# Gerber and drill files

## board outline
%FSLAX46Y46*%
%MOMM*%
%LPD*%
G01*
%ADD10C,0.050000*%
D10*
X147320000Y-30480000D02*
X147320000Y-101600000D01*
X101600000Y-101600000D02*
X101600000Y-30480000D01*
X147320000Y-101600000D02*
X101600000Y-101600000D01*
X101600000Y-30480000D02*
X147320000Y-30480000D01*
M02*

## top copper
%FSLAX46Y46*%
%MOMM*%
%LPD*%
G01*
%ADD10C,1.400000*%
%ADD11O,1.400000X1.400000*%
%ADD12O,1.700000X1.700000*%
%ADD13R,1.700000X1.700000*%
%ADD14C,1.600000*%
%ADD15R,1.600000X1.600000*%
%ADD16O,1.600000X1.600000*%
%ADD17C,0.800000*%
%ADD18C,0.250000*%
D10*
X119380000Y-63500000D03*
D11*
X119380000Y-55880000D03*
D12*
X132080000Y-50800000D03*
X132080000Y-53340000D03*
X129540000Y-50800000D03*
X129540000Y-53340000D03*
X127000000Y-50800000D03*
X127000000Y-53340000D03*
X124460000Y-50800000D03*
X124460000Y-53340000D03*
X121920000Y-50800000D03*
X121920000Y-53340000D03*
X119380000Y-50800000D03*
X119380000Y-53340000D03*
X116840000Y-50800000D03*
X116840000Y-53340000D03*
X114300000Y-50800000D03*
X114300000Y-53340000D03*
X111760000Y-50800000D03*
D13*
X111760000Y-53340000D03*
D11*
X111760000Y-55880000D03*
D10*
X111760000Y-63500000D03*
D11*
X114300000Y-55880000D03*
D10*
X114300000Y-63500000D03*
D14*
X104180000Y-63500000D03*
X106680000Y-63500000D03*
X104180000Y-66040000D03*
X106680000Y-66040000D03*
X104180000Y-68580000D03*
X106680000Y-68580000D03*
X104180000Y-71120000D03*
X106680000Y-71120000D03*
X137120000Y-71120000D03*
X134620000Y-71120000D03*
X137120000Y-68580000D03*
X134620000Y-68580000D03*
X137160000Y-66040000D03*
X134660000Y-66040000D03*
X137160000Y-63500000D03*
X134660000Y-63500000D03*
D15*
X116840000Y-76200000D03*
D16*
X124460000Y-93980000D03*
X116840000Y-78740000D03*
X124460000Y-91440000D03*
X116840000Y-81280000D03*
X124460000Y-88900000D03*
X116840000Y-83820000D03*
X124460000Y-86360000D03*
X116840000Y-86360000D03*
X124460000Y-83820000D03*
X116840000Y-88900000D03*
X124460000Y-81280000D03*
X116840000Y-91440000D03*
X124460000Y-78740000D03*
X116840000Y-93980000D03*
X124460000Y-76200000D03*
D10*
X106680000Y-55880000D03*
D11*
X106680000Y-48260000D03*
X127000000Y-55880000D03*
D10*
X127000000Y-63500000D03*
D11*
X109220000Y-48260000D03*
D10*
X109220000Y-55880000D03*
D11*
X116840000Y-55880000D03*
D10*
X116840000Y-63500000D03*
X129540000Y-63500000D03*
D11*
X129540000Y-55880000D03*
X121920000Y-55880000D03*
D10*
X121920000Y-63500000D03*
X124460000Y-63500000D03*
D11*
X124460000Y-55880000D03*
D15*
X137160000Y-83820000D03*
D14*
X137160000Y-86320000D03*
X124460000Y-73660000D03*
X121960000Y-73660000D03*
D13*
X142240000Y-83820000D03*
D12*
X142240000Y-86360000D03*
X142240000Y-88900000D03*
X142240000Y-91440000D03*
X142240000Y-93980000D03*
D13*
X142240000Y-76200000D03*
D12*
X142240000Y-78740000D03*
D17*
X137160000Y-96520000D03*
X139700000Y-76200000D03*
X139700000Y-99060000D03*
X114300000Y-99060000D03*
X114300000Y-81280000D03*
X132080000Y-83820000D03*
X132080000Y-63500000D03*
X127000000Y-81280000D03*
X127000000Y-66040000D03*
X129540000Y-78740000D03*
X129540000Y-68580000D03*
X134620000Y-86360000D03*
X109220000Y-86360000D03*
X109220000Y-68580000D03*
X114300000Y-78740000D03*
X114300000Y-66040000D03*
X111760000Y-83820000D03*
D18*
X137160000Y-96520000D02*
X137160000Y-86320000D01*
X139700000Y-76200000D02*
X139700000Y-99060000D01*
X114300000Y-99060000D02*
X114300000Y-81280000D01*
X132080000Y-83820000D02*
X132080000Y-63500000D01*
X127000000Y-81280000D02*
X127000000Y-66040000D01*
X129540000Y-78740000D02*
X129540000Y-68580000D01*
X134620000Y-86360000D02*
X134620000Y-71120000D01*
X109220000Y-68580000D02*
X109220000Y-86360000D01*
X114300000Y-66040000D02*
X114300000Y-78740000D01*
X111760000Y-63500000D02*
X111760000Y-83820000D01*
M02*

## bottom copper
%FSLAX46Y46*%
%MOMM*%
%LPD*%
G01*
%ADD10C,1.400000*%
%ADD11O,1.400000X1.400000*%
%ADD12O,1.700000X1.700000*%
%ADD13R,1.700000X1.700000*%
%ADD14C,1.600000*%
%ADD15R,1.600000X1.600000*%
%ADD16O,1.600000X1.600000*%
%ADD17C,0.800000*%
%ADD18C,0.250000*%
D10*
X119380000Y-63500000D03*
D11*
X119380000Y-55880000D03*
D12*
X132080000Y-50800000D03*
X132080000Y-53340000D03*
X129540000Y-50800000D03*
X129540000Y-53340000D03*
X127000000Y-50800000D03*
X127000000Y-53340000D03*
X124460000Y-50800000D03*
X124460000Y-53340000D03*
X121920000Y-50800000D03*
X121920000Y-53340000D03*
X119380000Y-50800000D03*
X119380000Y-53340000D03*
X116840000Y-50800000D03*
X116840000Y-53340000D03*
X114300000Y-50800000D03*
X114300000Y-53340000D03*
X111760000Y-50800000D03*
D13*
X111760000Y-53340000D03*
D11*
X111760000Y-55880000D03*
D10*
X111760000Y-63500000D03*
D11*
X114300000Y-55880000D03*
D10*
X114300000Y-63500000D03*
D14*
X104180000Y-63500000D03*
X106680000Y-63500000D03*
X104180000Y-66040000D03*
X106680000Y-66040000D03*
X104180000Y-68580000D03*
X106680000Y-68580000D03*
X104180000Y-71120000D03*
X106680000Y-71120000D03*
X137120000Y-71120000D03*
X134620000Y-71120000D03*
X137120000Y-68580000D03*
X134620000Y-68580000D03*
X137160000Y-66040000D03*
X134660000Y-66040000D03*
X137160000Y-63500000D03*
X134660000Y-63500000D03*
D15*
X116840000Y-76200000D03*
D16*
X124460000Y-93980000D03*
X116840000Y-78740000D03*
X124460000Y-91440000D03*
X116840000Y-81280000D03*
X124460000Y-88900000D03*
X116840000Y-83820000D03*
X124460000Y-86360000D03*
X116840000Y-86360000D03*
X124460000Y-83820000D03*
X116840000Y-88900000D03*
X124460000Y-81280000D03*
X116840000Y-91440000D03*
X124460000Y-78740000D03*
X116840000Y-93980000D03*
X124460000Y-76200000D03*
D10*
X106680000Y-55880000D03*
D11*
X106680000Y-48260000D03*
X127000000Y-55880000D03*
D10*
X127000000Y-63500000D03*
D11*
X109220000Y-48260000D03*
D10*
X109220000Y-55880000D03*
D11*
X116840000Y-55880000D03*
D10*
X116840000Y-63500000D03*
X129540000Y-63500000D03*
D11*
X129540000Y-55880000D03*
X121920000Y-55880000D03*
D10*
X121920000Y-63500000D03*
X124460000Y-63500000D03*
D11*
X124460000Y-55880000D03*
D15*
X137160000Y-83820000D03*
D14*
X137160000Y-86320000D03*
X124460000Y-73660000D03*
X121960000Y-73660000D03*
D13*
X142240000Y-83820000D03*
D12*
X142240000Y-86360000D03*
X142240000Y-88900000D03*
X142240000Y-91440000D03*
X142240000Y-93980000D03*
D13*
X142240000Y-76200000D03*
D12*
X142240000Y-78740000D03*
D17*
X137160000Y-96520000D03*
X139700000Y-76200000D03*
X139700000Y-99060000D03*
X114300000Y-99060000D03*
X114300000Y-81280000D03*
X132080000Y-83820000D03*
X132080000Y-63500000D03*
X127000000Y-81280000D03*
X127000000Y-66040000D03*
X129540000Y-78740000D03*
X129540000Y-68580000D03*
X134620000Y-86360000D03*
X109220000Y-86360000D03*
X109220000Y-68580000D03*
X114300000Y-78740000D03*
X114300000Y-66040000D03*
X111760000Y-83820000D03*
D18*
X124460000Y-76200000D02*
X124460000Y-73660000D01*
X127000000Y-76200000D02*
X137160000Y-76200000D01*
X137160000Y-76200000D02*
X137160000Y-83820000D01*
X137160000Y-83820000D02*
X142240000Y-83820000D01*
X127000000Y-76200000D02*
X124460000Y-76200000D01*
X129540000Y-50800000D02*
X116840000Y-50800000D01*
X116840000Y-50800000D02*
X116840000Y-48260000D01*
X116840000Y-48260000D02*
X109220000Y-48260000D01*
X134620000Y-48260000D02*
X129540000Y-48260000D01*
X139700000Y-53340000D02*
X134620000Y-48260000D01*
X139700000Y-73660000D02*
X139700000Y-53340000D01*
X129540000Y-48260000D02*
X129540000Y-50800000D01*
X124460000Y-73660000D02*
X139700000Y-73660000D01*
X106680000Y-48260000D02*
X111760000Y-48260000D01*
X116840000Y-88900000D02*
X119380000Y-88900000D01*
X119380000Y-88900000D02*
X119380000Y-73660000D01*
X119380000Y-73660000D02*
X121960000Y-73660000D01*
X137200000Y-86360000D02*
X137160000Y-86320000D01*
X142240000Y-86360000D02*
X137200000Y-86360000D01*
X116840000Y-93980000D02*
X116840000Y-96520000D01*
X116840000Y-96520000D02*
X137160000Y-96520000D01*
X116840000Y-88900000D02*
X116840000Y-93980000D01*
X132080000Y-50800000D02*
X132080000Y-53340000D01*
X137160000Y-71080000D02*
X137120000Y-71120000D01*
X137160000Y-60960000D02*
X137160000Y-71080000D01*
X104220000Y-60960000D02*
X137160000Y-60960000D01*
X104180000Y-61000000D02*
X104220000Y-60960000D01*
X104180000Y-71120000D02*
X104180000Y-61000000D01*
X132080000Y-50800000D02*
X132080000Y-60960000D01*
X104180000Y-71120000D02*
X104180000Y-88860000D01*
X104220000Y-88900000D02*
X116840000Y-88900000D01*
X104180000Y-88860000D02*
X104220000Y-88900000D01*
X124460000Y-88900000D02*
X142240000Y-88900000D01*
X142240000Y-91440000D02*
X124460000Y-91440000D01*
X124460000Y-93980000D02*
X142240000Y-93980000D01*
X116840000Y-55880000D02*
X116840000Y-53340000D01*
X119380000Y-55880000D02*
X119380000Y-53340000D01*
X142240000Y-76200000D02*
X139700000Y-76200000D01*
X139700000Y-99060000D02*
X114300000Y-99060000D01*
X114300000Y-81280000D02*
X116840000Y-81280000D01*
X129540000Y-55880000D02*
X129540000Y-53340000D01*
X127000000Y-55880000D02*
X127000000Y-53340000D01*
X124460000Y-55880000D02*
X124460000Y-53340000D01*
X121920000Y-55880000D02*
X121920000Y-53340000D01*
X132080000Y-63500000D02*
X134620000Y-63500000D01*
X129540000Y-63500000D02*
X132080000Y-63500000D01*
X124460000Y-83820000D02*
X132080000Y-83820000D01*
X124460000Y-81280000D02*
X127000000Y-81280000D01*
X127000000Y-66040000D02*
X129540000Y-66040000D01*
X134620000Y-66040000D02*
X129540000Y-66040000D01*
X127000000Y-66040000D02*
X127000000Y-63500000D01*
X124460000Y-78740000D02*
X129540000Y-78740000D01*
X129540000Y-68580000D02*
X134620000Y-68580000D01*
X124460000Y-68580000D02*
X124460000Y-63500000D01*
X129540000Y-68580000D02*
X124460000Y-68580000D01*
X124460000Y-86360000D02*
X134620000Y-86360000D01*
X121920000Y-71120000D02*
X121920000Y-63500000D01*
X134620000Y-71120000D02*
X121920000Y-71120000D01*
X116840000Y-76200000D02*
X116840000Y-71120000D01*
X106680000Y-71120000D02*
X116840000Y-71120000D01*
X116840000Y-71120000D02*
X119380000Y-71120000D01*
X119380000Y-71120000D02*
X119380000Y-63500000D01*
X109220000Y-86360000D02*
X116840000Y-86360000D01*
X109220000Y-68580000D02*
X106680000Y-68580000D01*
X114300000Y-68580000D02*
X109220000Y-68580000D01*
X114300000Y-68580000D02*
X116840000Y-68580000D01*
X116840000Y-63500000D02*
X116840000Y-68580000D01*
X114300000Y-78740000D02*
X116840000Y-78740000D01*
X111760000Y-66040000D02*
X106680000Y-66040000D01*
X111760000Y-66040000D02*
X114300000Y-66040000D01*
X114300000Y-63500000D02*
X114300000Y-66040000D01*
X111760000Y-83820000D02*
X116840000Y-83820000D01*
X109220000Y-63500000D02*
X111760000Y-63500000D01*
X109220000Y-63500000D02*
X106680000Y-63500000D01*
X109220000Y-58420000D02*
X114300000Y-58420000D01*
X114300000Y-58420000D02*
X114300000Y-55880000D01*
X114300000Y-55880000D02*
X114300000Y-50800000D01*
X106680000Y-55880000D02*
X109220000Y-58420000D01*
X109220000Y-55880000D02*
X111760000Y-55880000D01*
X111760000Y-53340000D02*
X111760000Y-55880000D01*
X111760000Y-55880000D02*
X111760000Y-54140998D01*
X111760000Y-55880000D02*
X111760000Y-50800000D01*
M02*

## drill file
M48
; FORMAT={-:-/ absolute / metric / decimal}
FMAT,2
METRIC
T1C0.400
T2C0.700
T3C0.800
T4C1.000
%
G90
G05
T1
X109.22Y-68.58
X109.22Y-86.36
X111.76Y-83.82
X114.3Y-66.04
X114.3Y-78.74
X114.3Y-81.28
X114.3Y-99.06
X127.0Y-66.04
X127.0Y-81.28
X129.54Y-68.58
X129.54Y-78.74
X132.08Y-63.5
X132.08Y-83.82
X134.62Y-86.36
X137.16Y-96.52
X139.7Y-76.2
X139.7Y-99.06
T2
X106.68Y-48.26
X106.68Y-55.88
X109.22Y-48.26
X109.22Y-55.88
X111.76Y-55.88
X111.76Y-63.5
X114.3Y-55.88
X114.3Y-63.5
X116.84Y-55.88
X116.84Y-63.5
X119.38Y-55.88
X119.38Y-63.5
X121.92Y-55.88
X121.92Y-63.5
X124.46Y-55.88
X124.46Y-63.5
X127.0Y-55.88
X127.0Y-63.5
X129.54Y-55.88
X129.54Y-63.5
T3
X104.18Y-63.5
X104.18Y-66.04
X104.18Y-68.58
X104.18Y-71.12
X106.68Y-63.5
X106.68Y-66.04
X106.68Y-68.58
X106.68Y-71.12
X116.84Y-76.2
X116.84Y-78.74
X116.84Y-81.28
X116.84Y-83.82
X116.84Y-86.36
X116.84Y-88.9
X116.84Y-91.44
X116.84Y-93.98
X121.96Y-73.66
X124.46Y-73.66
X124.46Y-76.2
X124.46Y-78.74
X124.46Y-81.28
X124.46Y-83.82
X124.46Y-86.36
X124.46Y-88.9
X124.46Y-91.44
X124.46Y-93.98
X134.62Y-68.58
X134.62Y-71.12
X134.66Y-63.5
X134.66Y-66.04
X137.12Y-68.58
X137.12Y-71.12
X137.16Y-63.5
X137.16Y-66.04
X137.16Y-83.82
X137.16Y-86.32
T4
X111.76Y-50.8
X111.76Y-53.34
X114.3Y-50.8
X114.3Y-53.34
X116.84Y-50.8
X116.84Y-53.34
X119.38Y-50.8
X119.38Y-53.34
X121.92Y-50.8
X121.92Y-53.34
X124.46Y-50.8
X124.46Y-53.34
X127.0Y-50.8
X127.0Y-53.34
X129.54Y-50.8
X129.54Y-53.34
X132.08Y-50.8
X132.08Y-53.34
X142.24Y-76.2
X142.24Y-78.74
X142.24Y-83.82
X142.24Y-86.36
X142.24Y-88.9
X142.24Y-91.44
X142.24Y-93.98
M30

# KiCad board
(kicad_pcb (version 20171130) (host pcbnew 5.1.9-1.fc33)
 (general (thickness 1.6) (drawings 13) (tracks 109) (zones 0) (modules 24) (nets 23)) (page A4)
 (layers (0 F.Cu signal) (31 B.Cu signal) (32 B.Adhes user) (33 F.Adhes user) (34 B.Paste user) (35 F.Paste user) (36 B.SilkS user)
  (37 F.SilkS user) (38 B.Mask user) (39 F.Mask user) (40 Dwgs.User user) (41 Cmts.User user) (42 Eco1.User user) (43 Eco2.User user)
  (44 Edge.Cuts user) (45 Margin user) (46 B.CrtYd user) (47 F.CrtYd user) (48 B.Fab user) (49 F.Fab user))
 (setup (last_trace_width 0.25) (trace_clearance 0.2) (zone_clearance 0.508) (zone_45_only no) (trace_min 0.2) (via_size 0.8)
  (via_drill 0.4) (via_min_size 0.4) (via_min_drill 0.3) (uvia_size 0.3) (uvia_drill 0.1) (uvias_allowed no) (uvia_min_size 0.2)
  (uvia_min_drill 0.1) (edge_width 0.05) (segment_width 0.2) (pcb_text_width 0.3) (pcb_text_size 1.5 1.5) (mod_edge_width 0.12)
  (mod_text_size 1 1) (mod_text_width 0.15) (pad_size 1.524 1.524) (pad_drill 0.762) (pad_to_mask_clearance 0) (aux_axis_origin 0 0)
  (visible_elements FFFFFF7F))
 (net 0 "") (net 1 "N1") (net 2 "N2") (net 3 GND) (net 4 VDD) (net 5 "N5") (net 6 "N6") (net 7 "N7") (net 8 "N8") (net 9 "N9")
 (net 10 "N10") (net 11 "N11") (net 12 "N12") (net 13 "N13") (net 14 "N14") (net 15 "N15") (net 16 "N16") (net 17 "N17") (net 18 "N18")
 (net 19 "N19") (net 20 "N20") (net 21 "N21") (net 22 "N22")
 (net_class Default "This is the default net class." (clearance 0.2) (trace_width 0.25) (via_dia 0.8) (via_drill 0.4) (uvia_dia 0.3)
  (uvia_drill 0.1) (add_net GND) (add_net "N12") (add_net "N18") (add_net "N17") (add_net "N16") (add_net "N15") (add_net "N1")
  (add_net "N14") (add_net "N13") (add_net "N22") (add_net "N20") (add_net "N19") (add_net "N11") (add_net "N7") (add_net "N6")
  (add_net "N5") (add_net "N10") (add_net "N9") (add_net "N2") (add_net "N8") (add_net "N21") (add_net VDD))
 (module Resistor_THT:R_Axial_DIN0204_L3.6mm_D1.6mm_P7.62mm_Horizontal (layer F.Cu) (at 119.38 63.5 90)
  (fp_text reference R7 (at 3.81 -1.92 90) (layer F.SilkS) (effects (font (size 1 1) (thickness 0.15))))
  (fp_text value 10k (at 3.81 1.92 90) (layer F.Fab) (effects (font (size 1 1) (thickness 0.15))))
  (pad 1 thru_hole circle (at 0 0 90) (size 1.4 1.4) (drill 0.7) (layers *.Cu *.Mask) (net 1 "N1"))
  (pad 2 thru_hole oval (at 7.62 0 90) (size 1.4 1.4) (drill 0.7) (layers *.Cu *.Mask) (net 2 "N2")))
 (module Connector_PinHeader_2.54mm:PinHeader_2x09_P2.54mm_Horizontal (layer F.Cu) (at 111.76 53.34 90)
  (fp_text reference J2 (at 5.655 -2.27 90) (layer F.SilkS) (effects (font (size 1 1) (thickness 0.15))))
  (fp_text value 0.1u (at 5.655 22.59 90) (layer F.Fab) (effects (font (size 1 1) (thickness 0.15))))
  (pad 18 thru_hole oval (at 2.54 20.32 90) (size 1.7 1.7) (drill 1) (layers *.Cu *.Mask) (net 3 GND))
  (pad 17 thru_hole oval (at 0 20.32 90) (size 1.7 1.7) (drill 1) (layers *.Cu *.Mask) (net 3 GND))
  (pad 16 thru_hole oval (at 2.54 17.78 90) (size 1.7 1.7) (drill 1) (layers *.Cu *.Mask) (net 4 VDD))
  (pad 15 thru_hole oval (at 0 17.78 90) (size 1.7 1.7) (drill 1) (layers *.Cu *.Mask) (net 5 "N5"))
  (pad 14 thru_hole oval (at 2.54 15.24 90) (size 1.7 1.7) (drill 1) (layers *.Cu *.Mask) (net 4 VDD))
  (pad 13 thru_hole oval (at 0 15.24 90) (size 1.7 1.7) (drill 1) (layers *.Cu *.Mask) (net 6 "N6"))
  (pad 12 thru_hole oval (at 2.54 12.7 90) (size 1.7 1.7) (drill 1) (layers *.Cu *.Mask) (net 4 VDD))
  (pad 11 thru_hole oval (at 0 12.7 90) (size 1.7 1.7) (drill 1) (layers *.Cu *.Mask) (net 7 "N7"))
  (pad 10 thru_hole oval (at 2.54 10.16 90) (size 1.7 1.7) (drill 1) (layers *.Cu *.Mask) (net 4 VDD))
  (pad 9 thru_hole oval (at 0 10.16 90) (size 1.7 1.7) (drill 1) (layers *.Cu *.Mask) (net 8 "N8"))
  (pad 8 thru_hole oval (at 2.54 7.62 90) (size 1.7 1.7) (drill 1) (layers *.Cu *.Mask) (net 4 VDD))
  (pad 7 thru_hole oval (at 0 7.62 90) (size 1.7 1.7) (drill 1) (layers *.Cu *.Mask) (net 2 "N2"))
  (pad 6 thru_hole oval (at 2.54 5.08 90) (size 1.7 1.7) (drill 1) (layers *.Cu *.Mask) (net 4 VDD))
  (pad 5 thru_hole oval (at 0 5.08 90) (size 1.7 1.7) (drill 1) (layers *.Cu *.Mask) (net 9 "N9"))
  (pad 4 thru_hole oval (at 2.54 2.54 90) (size 1.7 1.7) (drill 1) (layers *.Cu *.Mask) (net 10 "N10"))
  (pad 3 thru_hole oval (at 0 2.54 90) (size 1.7 1.7) (drill 1) (layers *.Cu *.Mask) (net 10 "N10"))
  (pad 2 thru_hole oval (at 2.54 0 90) (size 1.7 1.7) (drill 1) (layers *.Cu *.Mask) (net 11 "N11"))
  (pad 1 thru_hole rect (at 0 0 90) (size 1.7 1.7) (drill 1) (layers *.Cu *.Mask) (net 11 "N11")))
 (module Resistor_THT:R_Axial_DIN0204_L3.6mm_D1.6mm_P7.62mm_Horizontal (layer F.Cu) (at 111.76 63.5 90)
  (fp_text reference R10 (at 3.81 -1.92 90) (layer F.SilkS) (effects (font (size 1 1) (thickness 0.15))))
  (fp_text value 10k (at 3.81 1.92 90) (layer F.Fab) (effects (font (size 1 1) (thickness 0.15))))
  (pad 2 thru_hole oval (at 7.62 0 90) (size 1.4 1.4) (drill 0.7) (layers *.Cu *.Mask) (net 11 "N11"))
  (pad 1 thru_hole circle (at 0 0 90) (size 1.4 1.4) (drill 0.7) (layers *.Cu *.Mask) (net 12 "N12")))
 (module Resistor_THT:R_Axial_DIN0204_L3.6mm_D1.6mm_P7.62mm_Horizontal (layer F.Cu) (at 114.3 63.5 90)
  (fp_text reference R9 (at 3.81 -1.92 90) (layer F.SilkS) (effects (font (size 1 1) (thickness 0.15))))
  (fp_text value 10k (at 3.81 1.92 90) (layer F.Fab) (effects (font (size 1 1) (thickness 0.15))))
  (pad 2 thru_hole oval (at 7.62 0 90) (size 1.4 1.4) (drill 0.7) (layers *.Cu *.Mask) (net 10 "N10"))
  (pad 1 thru_hole circle (at 0 0 90) (size 1.4 1.4) (drill 0.7) (layers *.Cu *.Mask) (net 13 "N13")))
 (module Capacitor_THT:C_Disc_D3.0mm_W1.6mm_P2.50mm (layer F.Cu) (at 106.68 63.5 180)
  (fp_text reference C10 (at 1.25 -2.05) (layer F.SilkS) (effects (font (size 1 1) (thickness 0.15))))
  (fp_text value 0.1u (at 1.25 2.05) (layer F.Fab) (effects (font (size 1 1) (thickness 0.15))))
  (pad 2 thru_hole circle (at 2.5 0 180) (size 1.6 1.6) (drill 0.8) (layers *.Cu *.Mask) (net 3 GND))
  (pad 1 thru_hole circle (at 0 0 180) (size 1.6 1.6) (drill 0.8) (layers *.Cu *.Mask) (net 12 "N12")))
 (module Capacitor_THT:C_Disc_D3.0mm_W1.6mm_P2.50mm (layer F.Cu) (at 106.68 66.04 180)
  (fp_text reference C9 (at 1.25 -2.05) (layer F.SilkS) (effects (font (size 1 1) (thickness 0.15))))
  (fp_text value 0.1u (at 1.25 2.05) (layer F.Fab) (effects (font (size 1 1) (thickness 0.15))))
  (pad 2 thru_hole circle (at 2.5 0 180) (size 1.6 1.6) (drill 0.8) (layers *.Cu *.Mask) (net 3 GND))
  (pad 1 thru_hole circle (at 0 0 180) (size 1.6 1.6) (drill 0.8) (layers *.Cu *.Mask) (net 13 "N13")))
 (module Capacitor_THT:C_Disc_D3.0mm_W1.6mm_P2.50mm (layer F.Cu) (at 106.68 68.58 180)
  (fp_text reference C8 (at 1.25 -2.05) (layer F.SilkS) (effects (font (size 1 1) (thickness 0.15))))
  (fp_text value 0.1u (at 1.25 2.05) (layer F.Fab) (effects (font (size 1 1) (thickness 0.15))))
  (pad 2 thru_hole circle (at 2.5 0 180) (size 1.6 1.6) (drill 0.8) (layers *.Cu *.Mask) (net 3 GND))
  (pad 1 thru_hole circle (at 0 0 180) (size 1.6 1.6) (drill 0.8) (layers *.Cu *.Mask) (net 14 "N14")))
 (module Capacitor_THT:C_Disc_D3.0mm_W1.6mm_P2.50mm (layer F.Cu) (at 106.68 71.12 180)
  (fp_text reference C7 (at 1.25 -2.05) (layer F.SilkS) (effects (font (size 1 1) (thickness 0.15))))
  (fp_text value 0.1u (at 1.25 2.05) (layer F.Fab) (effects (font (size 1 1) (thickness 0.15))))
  (pad 2 thru_hole circle (at 2.5 0 180) (size 1.6 1.6) (drill 0.8) (layers *.Cu *.Mask) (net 3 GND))
  (pad 1 thru_hole circle (at 0 0 180) (size 1.6 1.6) (drill 0.8) (layers *.Cu *.Mask) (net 1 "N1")))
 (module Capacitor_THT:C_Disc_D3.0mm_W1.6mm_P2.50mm (layer F.Cu) (at 134.62 71.12)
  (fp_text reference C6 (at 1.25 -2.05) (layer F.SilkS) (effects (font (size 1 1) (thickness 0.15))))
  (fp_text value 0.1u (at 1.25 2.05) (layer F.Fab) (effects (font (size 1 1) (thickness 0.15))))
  (pad 2 thru_hole circle (at 2.5 0) (size 1.6 1.6) (drill 0.8) (layers *.Cu *.Mask) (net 3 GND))
  (pad 1 thru_hole circle (at 0 0) (size 1.6 1.6) (drill 0.8) (layers *.Cu *.Mask) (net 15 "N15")))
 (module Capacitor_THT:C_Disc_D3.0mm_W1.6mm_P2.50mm (layer F.Cu) (at 134.62 68.58)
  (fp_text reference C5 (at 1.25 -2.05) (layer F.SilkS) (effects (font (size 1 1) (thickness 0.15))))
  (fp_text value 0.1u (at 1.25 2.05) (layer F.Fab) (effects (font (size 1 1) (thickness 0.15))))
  (pad 2 thru_hole circle (at 2.5 0) (size 1.6 1.6) (drill 0.8) (layers *.Cu *.Mask) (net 3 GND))
  (pad 1 thru_hole circle (at 0 0) (size 1.6 1.6) (drill 0.8) (layers *.Cu *.Mask) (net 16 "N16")))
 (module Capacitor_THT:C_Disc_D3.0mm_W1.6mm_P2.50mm (layer F.Cu) (at 134.66 66.04)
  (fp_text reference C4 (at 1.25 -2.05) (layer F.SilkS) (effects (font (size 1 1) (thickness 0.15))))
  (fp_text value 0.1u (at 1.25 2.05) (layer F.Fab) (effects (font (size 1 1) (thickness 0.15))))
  (pad 2 thru_hole circle (at 2.5 0) (size 1.6 1.6) (drill 0.8) (layers *.Cu *.Mask) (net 3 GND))
  (pad 1 thru_hole circle (at 0 0) (size 1.6 1.6) (drill 0.8) (layers *.Cu *.Mask) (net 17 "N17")))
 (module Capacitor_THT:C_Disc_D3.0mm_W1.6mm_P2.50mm (layer F.Cu) (at 134.66 63.5)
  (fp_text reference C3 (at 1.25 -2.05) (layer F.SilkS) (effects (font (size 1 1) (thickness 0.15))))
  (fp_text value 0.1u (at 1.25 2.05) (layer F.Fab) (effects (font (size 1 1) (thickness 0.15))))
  (pad 2 thru_hole circle (at 2.5 0) (size 1.6 1.6) (drill 0.8) (layers *.Cu *.Mask) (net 3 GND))
  (pad 1 thru_hole circle (at 0 0) (size 1.6 1.6) (drill 0.8) (layers *.Cu *.Mask) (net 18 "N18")))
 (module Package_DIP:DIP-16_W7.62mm (layer F.Cu) (at 116.84 76.2)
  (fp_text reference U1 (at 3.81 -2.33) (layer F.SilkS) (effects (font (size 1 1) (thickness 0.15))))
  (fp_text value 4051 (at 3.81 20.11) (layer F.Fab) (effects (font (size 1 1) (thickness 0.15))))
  (pad 1 thru_hole rect (at 0 0) (size 1.6 1.6) (drill 0.8) (layers *.Cu *.Mask) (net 1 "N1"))
  (pad 9 thru_hole oval (at 7.62 17.78) (size 1.6 1.6) (drill 0.8) (layers *.Cu *.Mask) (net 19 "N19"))
  (pad 2 thru_hole oval (at 0 2.54) (size 1.6 1.6) (drill 0.8) (layers *.Cu *.Mask) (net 13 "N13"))
  (pad 10 thru_hole oval (at 7.62 15.24) (size 1.6 1.6) (drill 0.8) (layers *.Cu *.Mask) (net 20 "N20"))
  (pad 3 thru_hole oval (at 0 5.08) (size 1.6 1.6) (drill 0.8) (layers *.Cu *.Mask) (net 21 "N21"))
  (pad 11 thru_hole oval (at 7.62 12.7) (size 1.6 1.6) (drill 0.8) (layers *.Cu *.Mask) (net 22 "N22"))
  (pad 4 thru_hole oval (at 0 7.62) (size 1.6 1.6) (drill 0.8) (layers *.Cu *.Mask) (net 12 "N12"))
  (pad 12 thru_hole oval (at 7.62 10.16) (size 1.6 1.6) (drill 0.8) (layers *.Cu *.Mask) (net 15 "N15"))
  (pad 5 thru_hole oval (at 0 10.16) (size 1.6 1.6) (drill 0.8) (layers *.Cu *.Mask) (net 14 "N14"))
  (pad 13 thru_hole oval (at 7.62 7.62) (size 1.6 1.6) (drill 0.8) (layers *.Cu *.Mask) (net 18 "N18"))
  (pad 6 thru_hole oval (at 0 12.7) (size 1.6 1.6) (drill 0.8) (layers *.Cu *.Mask) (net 3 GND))
  (pad 14 thru_hole oval (at 7.62 5.08) (size 1.6 1.6) (drill 0.8) (layers *.Cu *.Mask) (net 17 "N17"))
  (pad 7 thru_hole oval (at 0 15.24) (size 1.6 1.6) (drill 0.8) (layers *.Cu *.Mask) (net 3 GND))
  (pad 15 thru_hole oval (at 7.62 2.54) (size 1.6 1.6) (drill 0.8) (layers *.Cu *.Mask) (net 16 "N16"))
  (pad 8 thru_hole oval (at 0 17.78) (size 1.6 1.6) (drill 0.8) (layers *.Cu *.Mask) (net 3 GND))
  (pad 16 thru_hole oval (at 7.62 0) (size 1.6 1.6) (drill 0.8) (layers *.Cu *.Mask) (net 4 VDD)))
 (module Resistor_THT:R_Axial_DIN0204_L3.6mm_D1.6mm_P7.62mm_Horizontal (layer F.Cu) (at 106.68 55.88 90)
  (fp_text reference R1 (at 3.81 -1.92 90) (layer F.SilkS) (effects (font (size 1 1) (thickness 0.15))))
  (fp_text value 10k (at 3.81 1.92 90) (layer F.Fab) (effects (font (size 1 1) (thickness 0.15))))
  (pad 1 thru_hole circle (at 0 0 90) (size 1.4 1.4) (drill 0.7) (layers *.Cu *.Mask) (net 10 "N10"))
  (pad 2 thru_hole oval (at 7.62 0 90) (size 1.4 1.4) (drill 0.7) (layers *.Cu *.Mask) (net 4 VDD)))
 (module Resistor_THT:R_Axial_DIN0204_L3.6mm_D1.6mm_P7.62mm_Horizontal (layer F.Cu) (at 127 63.5 90)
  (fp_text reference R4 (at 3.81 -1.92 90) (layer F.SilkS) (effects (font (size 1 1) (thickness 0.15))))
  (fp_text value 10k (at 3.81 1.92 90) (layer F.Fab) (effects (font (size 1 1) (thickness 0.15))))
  (pad 2 thru_hole oval (at 7.62 0 90) (size 1.4 1.4) (drill 0.7) (layers *.Cu *.Mask) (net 6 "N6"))
  (pad 1 thru_hole circle (at 0 0 90) (size 1.4 1.4) (drill 0.7) (layers *.Cu *.Mask) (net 17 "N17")))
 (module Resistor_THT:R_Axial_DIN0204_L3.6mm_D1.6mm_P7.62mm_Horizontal (layer F.Cu) (at 109.22 55.88 90)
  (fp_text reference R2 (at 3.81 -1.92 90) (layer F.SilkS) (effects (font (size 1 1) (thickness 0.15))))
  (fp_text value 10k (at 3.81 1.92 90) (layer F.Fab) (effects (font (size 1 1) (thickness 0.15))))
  (pad 2 thru_hole oval (at 7.62 0 90) (size 1.4 1.4) (drill 0.7) (layers *.Cu *.Mask) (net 4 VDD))
  (pad 1 thru_hole circle (at 0 0 90) (size 1.4 1.4) (drill 0.7) (layers *.Cu *.Mask) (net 11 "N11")))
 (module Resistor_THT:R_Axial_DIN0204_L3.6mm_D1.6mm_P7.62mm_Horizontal (layer F.Cu) (at 116.84 63.5 90)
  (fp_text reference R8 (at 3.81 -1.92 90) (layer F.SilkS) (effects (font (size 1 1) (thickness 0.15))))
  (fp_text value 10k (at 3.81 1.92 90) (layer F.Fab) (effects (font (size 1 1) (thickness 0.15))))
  (pad 2 thru_hole oval (at 7.62 0 90) (size 1.4 1.4) (drill 0.7) (layers *.Cu *.Mask) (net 9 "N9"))
  (pad 1 thru_hole circle (at 0 0 90) (size 1.4 1.4) (drill 0.7) (layers *.Cu *.Mask) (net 14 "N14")))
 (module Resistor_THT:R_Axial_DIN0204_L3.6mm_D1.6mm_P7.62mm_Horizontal (layer F.Cu) (at 129.54 63.5 90)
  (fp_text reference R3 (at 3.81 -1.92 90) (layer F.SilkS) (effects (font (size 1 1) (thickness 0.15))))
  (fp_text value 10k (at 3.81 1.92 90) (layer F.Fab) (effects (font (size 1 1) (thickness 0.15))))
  (pad 1 thru_hole circle (at 0 0 90) (size 1.4 1.4) (drill 0.7) (layers *.Cu *.Mask) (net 18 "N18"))
  (pad 2 thru_hole oval (at 7.62 0 90) (size 1.4 1.4) (drill 0.7) (layers *.Cu *.Mask) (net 5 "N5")))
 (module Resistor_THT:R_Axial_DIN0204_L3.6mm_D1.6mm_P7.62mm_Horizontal (layer F.Cu) (at 121.92 63.5 90)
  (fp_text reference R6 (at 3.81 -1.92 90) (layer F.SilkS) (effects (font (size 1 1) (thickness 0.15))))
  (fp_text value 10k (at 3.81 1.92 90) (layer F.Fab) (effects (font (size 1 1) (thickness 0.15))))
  (pad 2 thru_hole oval (at 7.62 0 90) (size 1.4 1.4) (drill 0.7) (layers *.Cu *.Mask) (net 8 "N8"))
  (pad 1 thru_hole circle (at 0 0 90) (size 1.4 1.4) (drill 0.7) (layers *.Cu *.Mask) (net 15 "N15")))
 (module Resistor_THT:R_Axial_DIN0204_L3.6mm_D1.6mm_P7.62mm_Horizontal (layer F.Cu) (at 124.46 63.5 90)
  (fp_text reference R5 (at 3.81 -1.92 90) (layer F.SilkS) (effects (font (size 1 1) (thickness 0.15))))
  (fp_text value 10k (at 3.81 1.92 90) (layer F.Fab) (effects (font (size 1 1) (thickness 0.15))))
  (pad 1 thru_hole circle (at 0 0 90) (size 1.4 1.4) (drill 0.7) (layers *.Cu *.Mask) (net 16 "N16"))
  (pad 2 thru_hole oval (at 7.62 0 90) (size 1.4 1.4) (drill 0.7) (layers *.Cu *.Mask) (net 7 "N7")))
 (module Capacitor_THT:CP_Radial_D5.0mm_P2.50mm (layer F.Cu) (at 137.16 83.82 270)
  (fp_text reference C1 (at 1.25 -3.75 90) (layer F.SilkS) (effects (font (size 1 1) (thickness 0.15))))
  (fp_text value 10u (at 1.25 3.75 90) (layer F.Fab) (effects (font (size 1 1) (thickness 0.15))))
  (pad 1 thru_hole rect (at 0 0 270) (size 1.6 1.6) (drill 0.8) (layers *.Cu *.Mask) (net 4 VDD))
  (pad 2 thru_hole circle (at 2.5 0 270) (size 1.6 1.6) (drill 0.8) (layers *.Cu *.Mask) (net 3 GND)))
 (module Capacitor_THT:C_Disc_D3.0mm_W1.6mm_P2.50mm (layer F.Cu) (at 124.46 73.66 180)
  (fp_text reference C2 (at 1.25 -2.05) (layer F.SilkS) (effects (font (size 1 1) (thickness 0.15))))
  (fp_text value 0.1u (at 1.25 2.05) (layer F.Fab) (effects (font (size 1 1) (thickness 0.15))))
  (pad 1 thru_hole circle (at 0 0 180) (size 1.6 1.6) (drill 0.8) (layers *.Cu *.Mask) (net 4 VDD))
  (pad 2 thru_hole circle (at 2.5 0 180) (size 1.6 1.6) (drill 0.8) (layers *.Cu *.Mask) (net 3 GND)))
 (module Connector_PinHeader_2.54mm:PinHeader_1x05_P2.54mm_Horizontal (layer F.Cu) (at 142.24 83.82)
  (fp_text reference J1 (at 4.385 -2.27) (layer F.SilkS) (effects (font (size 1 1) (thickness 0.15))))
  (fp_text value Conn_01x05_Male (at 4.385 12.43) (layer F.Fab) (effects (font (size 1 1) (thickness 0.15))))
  (pad 1 thru_hole rect (at 0 0) (size 1.7 1.7) (drill 1) (layers *.Cu *.Mask) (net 4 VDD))
  (pad 2 thru_hole oval (at 0 2.54) (size 1.7 1.7) (drill 1) (layers *.Cu *.Mask) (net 3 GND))
  (pad 3 thru_hole oval (at 0 5.08) (size 1.7 1.7) (drill 1) (layers *.Cu *.Mask) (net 22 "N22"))
  (pad 4 thru_hole oval (at 0 7.62) (size 1.7 1.7) (drill 1) (layers *.Cu *.Mask) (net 20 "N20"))
  (pad 5 thru_hole oval (at 0 10.16) (size 1.7 1.7) (drill 1) (layers *.Cu *.Mask) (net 19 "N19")))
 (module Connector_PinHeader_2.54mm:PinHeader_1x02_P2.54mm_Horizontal (layer F.Cu) (at 142.24 76.2)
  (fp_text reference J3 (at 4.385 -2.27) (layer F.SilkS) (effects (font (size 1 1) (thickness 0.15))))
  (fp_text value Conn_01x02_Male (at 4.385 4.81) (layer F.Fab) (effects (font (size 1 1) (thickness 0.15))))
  (pad 1 thru_hole rect (at 0 0) (size 1.7 1.7) (drill 1) (layers *.Cu *.Mask) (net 21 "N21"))
  (pad 2 thru_hole oval (at 0 2.54) (size 1.7 1.7) (drill 1) (layers *.Cu *.Mask)))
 (gr_line (start 147.32 30.48) (end 147.32 101.6) (layer Edge.Cuts) (width 0.05))
 (gr_line (start 101.6 101.6) (end 101.6 30.48) (layer Edge.Cuts) (width 0.05))
 (gr_line (start 147.32 101.6) (end 101.6 101.6) (layer Edge.Cuts) (width 0.05))
 (gr_line (start 101.6 30.48) (end 147.32 30.48) (layer Edge.Cuts) (width 0.05))
 (segment (start 124.46 76.2) (end 124.46 73.66) (width 0.25) (layer B.Cu) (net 4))
 (segment (start 127 76.2) (end 137.16 76.2) (width 0.25) (layer B.Cu) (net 4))
 (segment (start 137.16 76.2) (end 137.16 83.82) (width 0.25) (layer B.Cu) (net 4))
 (segment (start 137.16 83.82) (end 142.24 83.82) (width 0.25) (layer B.Cu) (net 4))
 (segment (start 127 76.2) (end 124.46 76.2) (width 0.25) (layer B.Cu) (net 4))
 (segment (start 129.54 50.8) (end 116.84 50.8) (width 0.25) (layer B.Cu) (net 4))
 (segment (start 116.84 50.8) (end 116.84 48.26) (width 0.25) (layer B.Cu) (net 4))
 (segment (start 116.84 48.26) (end 109.22 48.26) (width 0.25) (layer B.Cu) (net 4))
 (segment (start 134.62 48.26) (end 129.54 48.26) (width 0.25) (layer B.Cu) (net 4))
 (segment (start 139.7 53.34) (end 134.62 48.26) (width 0.25) (layer B.Cu) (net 4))
 (segment (start 139.7 73.66) (end 139.7 53.34) (width 0.25) (layer B.Cu) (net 4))
 (segment (start 129.54 48.26) (end 129.54 50.8) (width 0.25) (layer B.Cu) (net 4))
 (segment (start 124.46 73.66) (end 139.7 73.66) (width 0.25) (layer B.Cu) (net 4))
 (segment (start 106.68 48.26) (end 111.76 48.26) (width 0.25) (layer B.Cu) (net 4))
 (segment (start 116.84 88.9) (end 119.38 88.9) (width 0.25) (layer B.Cu) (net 3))
 (segment (start 119.38 88.9) (end 119.38 73.66) (width 0.25) (layer B.Cu) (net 3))
 (segment (start 119.38 73.66) (end 121.96 73.66) (width 0.25) (layer B.Cu) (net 3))
 (segment (start 137.2 86.36) (end 137.16 86.32) (width 0.25) (layer B.Cu) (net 3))
 (segment (start 142.24 86.36) (end 137.2 86.36) (width 0.25) (layer B.Cu) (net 3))
 (segment (start 116.84 93.98) (end 116.84 96.52) (width 0.25) (layer B.Cu) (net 3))
 (via (at 137.16 96.52) (size 0.8) (drill 0.4) (layers F.Cu B.Cu) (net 3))
 (segment (start 116.84 96.52) (end 137.16 96.52) (width 0.25) (layer B.Cu) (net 3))
 (segment (start 137.16 96.52) (end 137.16 86.32) (width 0.25) (layer F.Cu) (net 3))
 (segment (start 116.84 88.9) (end 116.84 93.98) (width 0.25) (layer B.Cu) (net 3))
 (segment (start 132.08 50.8) (end 132.08 53.34) (width 0.25) (layer B.Cu) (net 3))
 (segment (start 137.16 71.08) (end 137.12 71.12) (width 0.25) (layer B.Cu) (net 3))
 (segment (start 137.16 60.96) (end 137.16 71.08) (width 0.25) (layer B.Cu) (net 3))
 (segment (start 104.22 60.96) (end 137.16 60.96) (width 0.25) (layer B.Cu) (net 3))
 (segment (start 104.18 61) (end 104.22 60.96) (width 0.25) (layer B.Cu) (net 3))
 (segment (start 104.18 71.12) (end 104.18 61) (width 0.25) (layer B.Cu) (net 3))
 (segment (start 132.08 50.8) (end 132.08 60.96) (width 0.25) (layer B.Cu) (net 3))
 (segment (start 104.18 71.12) (end 104.18 88.86) (width 0.25) (layer B.Cu) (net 3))
 (segment (start 104.22 88.9) (end 116.84 88.9) (width 0.25) (layer B.Cu) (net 3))
 (segment (start 104.18 88.86) (end 104.22 88.9) (width 0.25) (layer B.Cu) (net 3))
 (segment (start 124.46 88.9) (end 142.24 88.9) (width 0.25) (layer B.Cu) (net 22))
 (segment (start 142.24 91.44) (end 124.46 91.44) (width 0.25) (layer B.Cu) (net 20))
 (segment (start 124.46 93.98) (end 142.24 93.98) (width 0.25) (layer B.Cu) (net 19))
 (segment (start 116.84 55.88) (end 116.84 53.34) (width 0.25) (layer B.Cu) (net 9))
 (segment (start 119.38 55.88) (end 119.38 53.34) (width 0.25) (layer B.Cu) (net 2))
 (via (at 139.7 76.2) (size 0.8) (drill 0.4) (layers F.Cu B.Cu) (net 21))
 (segment (start 142.24 76.2) (end 139.7 76.2) (width 0.25) (layer B.Cu) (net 21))
 (via (at 139.7 99.06) (size 0.8) (drill 0.4) (layers F.Cu B.Cu) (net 21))
 (segment (start 139.7 76.2) (end 139.7 99.06) (width 0.25) (layer F.Cu) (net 21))
 (via (at 114.3 99.06) (size 0.8) (drill 0.4) (layers F.Cu B.Cu) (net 21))
 (segment (start 139.7 99.06) (end 114.3 99.06) (width 0.25) (layer B.Cu) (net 21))
 (via (at 114.3 81.28) (size 0.8) (drill 0.4) (layers F.Cu B.Cu) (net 21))
 (segment (start 114.3 99.06) (end 114.3 81.28) (width 0.25) (layer F.Cu) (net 21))
 (segment (start 114.3 81.28) (end 116.84 81.28) (width 0.25) (layer B.Cu) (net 21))
 (segment (start 129.54 55.88) (end 129.54 53.34) (width 0.25) (layer B.Cu) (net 5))
 (segment (start 127 55.88) (end 127 53.34) (width 0.25) (layer B.Cu) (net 6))
 (segment (start 124.46 55.88) (end 124.46 53.34) (width 0.25) (layer B.Cu) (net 7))
 (segment (start 121.92 55.88) (end 121.92 53.34) (width 0.25) (layer B.Cu) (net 8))
 (segment (start 132.08 63.5) (end 134.62 63.5) (width 0.25) (layer B.Cu) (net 18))
 (segment (start 129.54 63.5) (end 132.08 63.5) (width 0.25) (layer B.Cu) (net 18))
 (via (at 132.08 83.82) (size 0.8) (drill 0.4) (layers F.Cu B.Cu) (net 18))
 (segment (start 124.46 83.82) (end 132.08 83.82) (width 0.25) (layer B.Cu) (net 18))
 (segment (start 132.08 83.82) (end 132.08 63.5) (width 0.25) (layer F.Cu) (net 18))
 (via (at 132.08 63.5) (size 0.8) (drill 0.4) (layers F.Cu B.Cu) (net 18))
 (via (at 127 81.28) (size 0.8) (drill 0.4) (layers F.Cu B.Cu) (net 17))
 (segment (start 124.46 81.28) (end 127 81.28) (width 0.25) (layer B.Cu) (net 17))
 (segment (start 127 66.04) (end 129.54 66.04) (width 0.25) (layer B.Cu) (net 17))
 (segment (start 134.62 66.04) (end 129.54 66.04) (width 0.25) (layer B.Cu) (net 17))
 (via (at 127 66.04) (size 0.8) (drill 0.4) (layers F.Cu B.Cu) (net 17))
 (segment (start 127 81.28) (end 127 66.04) (width 0.25) (layer F.Cu) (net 17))
 (segment (start 127 66.04) (end 127 63.5) (width 0.25) (layer B.Cu) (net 17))
 (via (at 129.54 78.74) (size 0.8) (drill 0.4) (layers F.Cu B.Cu) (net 16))
 (segment (start 124.46 78.74) (end 129.54 78.74) (width 0.25) (layer B.Cu) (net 16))
 (segment (start 129.54 68.58) (end 134.62 68.58) (width 0.25) (layer B.Cu) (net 16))
 (segment (start 129.54 78.74) (end 129.54 68.58) (width 0.25) (layer F.Cu) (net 16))
 (via (at 129.54 68.58) (size 0.8) (drill 0.4) (layers F.Cu B.Cu) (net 16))
 (segment (start 124.46 68.58) (end 124.46 63.5) (width 0.25) (layer B.Cu) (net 16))
 (segment (start 129.54 68.58) (end 124.46 68.58) (width 0.25) (layer B.Cu) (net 16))
 (segment (start 124.46 86.36) (end 134.62 86.36) (width 0.25) (layer B.Cu) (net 15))
 (via (at 134.62 86.36) (size 0.8) (drill 0.4) (layers F.Cu B.Cu) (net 15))
 (segment (start 134.62 86.36) (end 134.62 71.12) (width 0.25) (layer F.Cu) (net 15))
 (segment (start 121.92 71.12) (end 121.92 63.5) (width 0.25) (layer B.Cu) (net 15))
 (segment (start 134.62 71.12) (end 121.92 71.12) (width 0.25) (layer B.Cu) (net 15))
 (segment (start 116.84 76.2) (end 116.84 71.12) (width 0.25) (layer B.Cu) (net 1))
 (segment (start 106.68 71.12) (end 116.84 71.12) (width 0.25) (layer B.Cu) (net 1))
 (segment (start 116.84 71.12) (end 119.38 71.12) (width 0.25) (layer B.Cu) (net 1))
 (segment (start 119.38 71.12) (end 119.38 63.5) (width 0.25) (layer B.Cu) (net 1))
 (via (at 109.22 86.36) (size 0.8) (drill 0.4) (layers F.Cu B.Cu) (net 14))
 (segment (start 109.22 86.36) (end 116.84 86.36) (width 0.25) (layer B.Cu) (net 14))
 (segment (start 109.22 68.58) (end 109.22 86.36) (width 0.25) (layer F.Cu) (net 14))
 (segment (start 109.22 68.58) (end 106.68 68.58) (width 0.25) (layer B.Cu) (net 14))
 (segment (start 114.3 68.58) (end 109.22 68.58) (width 0.25) (layer B.Cu) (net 14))
 (via (at 109.22 68.58) (size 0.8) (drill 0.4) (layers F.Cu B.Cu) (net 14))
 (segment (start 114.3 68.58) (end 116.84 68.58) (width 0.25) (layer B.Cu) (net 14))
 (segment (start 116.84 63.5) (end 116.84 68.58) (width 0.25) (layer B.Cu) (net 14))
 (via (at 114.3 78.74) (size 0.8) (drill 0.4) (layers F.Cu B.Cu) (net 13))
 (segment (start 114.3 78.74) (end 116.84 78.74) (width 0.25) (layer B.Cu) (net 13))
 (segment (start 111.76 66.04) (end 106.68 66.04) (width 0.25) (layer B.Cu) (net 13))
 (segment (start 114.3 66.04) (end 114.3 78.74) (width 0.25) (layer F.Cu) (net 13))
 (via (at 114.3 66.04) (size 0.8) (drill 0.4) (layers F.Cu B.Cu) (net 13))
 (segment (start 111.76 66.04) (end 114.3 66.04) (width 0.25) (layer B.Cu) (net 13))
 (segment (start 114.3 63.5) (end 114.3 66.04) (width 0.25) (layer B.Cu) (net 13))
 (via (at 111.76 83.82) (size 0.8) (drill 0.4) (layers F.Cu B.Cu) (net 12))
 (segment (start 111.76 83.82) (end 116.84 83.82) (width 0.25) (layer B.Cu) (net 12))
 (segment (start 111.76 63.5) (end 111.76 83.82) (width 0.25) (layer F.Cu) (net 12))
 (segment (start 109.22 63.5) (end 111.76 63.5) (width 0.25) (layer B.Cu) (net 12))
 (segment (start 109.22 63.5) (end 106.68 63.5) (width 0.25) (layer B.Cu) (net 12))
 (segment (start 109.22 58.42) (end 114.3 58.42) (width 0.25) (layer B.Cu) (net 10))
 (segment (start 114.3 58.42) (end 114.3 55.88) (width 0.25) (layer B.Cu) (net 10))
 (segment (start 114.3 55.88) (end 114.3 50.8) (width 0.25) (layer B.Cu) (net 10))
 (segment (start 106.68 55.88) (end 109.22 58.42) (width 0.25) (layer B.Cu) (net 10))
 (segment (start 109.22 55.88) (end 111.76 55.88) (width 0.25) (layer B.Cu) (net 11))
 (segment (start 111.76 53.34) (end 111.76 55.88) (width 0.25) (layer B.Cu) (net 11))
 (segment (start 111.76 55.88) (end 111.76 54.140998) (width 0.25) (layer B.Cu) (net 11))
 (segment (start 111.76 55.88) (end 111.76 50.8) (width 0.25) (layer B.Cu) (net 11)))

